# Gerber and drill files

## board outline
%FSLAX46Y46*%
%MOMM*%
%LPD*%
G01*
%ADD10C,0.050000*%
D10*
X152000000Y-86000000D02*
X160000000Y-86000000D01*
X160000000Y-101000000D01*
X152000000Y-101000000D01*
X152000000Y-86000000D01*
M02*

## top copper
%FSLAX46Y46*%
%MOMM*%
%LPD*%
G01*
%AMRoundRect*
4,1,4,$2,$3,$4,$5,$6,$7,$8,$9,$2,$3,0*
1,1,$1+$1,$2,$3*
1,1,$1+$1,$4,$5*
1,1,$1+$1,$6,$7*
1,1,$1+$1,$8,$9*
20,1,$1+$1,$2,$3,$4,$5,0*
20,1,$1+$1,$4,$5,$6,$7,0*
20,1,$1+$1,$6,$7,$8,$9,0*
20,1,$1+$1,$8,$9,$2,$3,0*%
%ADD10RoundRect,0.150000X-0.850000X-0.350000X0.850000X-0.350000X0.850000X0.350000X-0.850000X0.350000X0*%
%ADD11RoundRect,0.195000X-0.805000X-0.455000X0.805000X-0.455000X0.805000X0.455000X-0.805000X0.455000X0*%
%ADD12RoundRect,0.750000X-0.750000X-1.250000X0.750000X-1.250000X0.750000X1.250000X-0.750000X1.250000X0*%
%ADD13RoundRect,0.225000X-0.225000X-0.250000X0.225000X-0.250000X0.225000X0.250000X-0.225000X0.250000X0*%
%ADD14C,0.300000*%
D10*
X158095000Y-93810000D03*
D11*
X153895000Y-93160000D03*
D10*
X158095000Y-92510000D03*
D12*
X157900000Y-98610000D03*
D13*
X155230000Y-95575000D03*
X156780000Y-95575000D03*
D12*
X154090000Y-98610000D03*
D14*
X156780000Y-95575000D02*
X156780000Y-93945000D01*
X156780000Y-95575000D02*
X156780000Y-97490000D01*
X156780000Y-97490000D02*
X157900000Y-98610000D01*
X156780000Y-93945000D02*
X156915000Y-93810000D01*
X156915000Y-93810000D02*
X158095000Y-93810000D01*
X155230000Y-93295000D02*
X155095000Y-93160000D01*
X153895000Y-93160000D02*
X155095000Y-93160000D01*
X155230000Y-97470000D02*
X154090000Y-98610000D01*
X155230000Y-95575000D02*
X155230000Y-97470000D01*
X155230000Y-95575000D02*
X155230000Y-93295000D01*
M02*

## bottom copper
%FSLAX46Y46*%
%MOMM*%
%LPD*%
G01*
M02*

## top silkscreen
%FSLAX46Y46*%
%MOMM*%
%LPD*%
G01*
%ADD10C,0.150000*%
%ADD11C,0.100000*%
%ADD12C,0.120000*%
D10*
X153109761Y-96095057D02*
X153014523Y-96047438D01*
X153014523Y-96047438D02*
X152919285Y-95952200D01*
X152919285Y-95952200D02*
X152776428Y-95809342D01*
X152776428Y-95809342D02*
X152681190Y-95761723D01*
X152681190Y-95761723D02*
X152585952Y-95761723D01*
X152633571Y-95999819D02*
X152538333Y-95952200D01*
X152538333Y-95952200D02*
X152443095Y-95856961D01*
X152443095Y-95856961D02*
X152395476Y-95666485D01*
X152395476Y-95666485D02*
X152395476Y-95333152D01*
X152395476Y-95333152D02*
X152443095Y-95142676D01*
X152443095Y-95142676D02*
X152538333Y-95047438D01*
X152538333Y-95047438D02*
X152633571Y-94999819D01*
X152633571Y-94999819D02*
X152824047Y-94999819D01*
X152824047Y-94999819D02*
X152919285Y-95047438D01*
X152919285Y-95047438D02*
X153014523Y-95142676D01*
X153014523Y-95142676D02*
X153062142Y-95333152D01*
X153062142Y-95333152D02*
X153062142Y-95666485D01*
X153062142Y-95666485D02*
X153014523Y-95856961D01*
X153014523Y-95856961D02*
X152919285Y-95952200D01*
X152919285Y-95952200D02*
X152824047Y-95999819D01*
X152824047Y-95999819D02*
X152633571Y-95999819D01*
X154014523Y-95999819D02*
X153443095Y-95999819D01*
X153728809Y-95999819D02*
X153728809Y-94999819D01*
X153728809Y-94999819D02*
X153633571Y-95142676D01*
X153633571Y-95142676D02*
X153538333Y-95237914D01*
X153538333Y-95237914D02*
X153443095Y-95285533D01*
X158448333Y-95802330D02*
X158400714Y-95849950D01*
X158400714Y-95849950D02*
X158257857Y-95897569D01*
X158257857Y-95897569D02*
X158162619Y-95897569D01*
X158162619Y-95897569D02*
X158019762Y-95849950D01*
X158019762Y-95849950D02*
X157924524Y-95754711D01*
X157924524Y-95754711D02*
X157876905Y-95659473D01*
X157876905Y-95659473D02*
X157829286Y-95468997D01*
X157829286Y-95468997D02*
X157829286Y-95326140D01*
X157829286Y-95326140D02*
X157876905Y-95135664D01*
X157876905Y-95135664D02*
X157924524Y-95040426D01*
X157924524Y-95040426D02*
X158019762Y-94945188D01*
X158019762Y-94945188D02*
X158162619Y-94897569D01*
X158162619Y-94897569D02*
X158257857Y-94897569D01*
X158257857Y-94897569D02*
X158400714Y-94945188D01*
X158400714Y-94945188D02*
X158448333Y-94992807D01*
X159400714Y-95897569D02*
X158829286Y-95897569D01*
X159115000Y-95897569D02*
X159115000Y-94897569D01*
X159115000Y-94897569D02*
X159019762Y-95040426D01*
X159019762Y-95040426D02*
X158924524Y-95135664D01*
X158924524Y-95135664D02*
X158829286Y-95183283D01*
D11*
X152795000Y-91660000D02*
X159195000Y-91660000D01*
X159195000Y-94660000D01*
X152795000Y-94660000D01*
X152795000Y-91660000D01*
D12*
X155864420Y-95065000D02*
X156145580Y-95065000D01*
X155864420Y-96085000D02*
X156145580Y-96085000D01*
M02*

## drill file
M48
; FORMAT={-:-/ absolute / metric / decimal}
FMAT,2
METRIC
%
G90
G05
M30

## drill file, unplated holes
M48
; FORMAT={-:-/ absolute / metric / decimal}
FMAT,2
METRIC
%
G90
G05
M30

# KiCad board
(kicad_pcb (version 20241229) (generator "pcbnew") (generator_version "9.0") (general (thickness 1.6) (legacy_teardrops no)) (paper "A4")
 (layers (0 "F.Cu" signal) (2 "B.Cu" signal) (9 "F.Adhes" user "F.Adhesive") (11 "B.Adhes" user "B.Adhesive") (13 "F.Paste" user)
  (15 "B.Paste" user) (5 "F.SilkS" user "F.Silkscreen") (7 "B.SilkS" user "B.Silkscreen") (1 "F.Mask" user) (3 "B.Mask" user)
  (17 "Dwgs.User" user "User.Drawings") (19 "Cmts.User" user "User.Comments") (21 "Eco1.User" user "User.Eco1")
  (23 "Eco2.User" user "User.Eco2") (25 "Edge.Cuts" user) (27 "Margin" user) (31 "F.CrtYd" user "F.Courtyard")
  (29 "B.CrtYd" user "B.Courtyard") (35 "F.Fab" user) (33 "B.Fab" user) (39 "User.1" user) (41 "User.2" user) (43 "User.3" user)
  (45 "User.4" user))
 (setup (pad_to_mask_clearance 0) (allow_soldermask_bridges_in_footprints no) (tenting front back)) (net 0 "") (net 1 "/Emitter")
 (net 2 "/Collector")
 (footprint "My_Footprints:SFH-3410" (layer "F.Cu") (at 156.005 93.18)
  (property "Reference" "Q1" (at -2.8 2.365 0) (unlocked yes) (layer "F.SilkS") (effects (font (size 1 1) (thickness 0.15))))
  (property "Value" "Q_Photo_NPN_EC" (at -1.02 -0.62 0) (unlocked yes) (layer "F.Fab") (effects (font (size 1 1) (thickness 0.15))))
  (fp_rect (start -3.21 -1.52) (end 3.19 1.48) (stroke (width 0.1) (type solid)) (fill no) (layer "F.SilkS"))
  (pad "1" smd roundrect (at 2.09 0.63) (size 2 1) (layers "F.Cu" "F.Mask" "F.Paste") (roundrect_rratio 0.15) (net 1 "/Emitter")
   (thermal_bridge_angle 45))
  (pad "2" smd roundrect (at -2.11 -0.02) (size 2 1.3) (layers "F.Cu" "F.Mask" "F.Paste") (roundrect_rratio 0.15) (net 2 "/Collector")
   (thermal_bridge_angle 45))
  (pad "3" smd roundrect (at 2.09 -0.67) (size 2 1) (layers "F.Cu" "F.Mask" "F.Paste") (roundrect_rratio 0.15) (thermal_bridge_angle 45)))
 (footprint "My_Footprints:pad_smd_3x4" (layer "F.Cu") (at 158.1 98.61 -90)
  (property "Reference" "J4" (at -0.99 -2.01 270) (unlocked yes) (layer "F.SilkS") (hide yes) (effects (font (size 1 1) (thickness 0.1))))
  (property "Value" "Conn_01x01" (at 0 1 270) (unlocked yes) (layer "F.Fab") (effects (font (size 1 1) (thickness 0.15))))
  (pad "1" smd roundrect (at 0 0.2) (size 3 4) (layers "F.Cu" "F.Mask" "F.Paste") (roundrect_rratio 0.25) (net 1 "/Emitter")
   (thermal_bridge_angle 45)))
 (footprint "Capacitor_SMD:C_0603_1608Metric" (layer "F.Cu") (at 156.005 95.575)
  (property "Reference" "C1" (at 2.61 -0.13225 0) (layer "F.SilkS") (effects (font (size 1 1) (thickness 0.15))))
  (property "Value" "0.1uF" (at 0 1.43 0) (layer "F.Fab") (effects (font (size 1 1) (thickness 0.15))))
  (fp_line (start -0.14058 -0.51) (end 0.14058 -0.51) (stroke (width 0.12) (type solid)) (layer "F.SilkS"))
  (fp_line (start -0.14058 0.51) (end 0.14058 0.51) (stroke (width 0.12) (type solid)) (layer "F.SilkS"))
  (pad "1" smd roundrect (at -0.775 0) (size 0.9 0.95) (layers "F.Cu" "F.Mask" "F.Paste") (roundrect_rratio 0.25) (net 2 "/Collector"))
  (pad "2" smd roundrect (at 0.775 0) (size 0.9 0.95) (layers "F.Cu" "F.Mask" "F.Paste") (roundrect_rratio 0.25) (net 1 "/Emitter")))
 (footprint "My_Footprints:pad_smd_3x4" (layer "F.Cu") (at 154.29 98.61 -90)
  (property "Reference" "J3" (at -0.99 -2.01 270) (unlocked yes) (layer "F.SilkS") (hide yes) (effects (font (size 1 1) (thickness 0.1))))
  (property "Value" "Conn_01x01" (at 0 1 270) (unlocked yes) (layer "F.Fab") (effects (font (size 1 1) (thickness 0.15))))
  (pad "1" smd roundrect (at 0 0.2) (size 3 4) (layers "F.Cu" "F.Mask" "F.Paste") (roundrect_rratio 0.25) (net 2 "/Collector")
   (thermal_bridge_angle 45)))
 (gr_rect (start 152 86) (end 160 101) (stroke (width 0.05) (type solid)) (fill no) (layer "Edge.Cuts"))
 (segment (start 156.78 95.575) (end 156.78 93.945) (width 0.3) (layer "F.Cu") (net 1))
 (segment (start 156.78 95.575) (end 156.78 97.49) (width 0.3) (layer "F.Cu") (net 1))
 (segment (start 156.78 97.49) (end 157.9 98.61) (width 0.3) (layer "F.Cu") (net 1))
 (segment (start 156.78 93.945) (end 156.915 93.81) (width 0.3) (layer "F.Cu") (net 1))
 (segment (start 156.915 93.81) (end 158.095 93.81) (width 0.3) (layer "F.Cu") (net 1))
 (segment (start 155.23 93.295) (end 155.095 93.16) (width 0.3) (layer "F.Cu") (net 2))
 (segment (start 153.895 93.16) (end 155.095 93.16) (width 0.3) (layer "F.Cu") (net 2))
 (segment (start 155.23 97.47) (end 154.09 98.61) (width 0.3) (layer "F.Cu") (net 2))
 (segment (start 155.23 95.575) (end 155.23 97.47) (width 0.3) (layer "F.Cu") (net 2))
 (segment (start 155.23 95.575) (end 155.23 93.295) (width 0.3) (layer "F.Cu") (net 2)))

